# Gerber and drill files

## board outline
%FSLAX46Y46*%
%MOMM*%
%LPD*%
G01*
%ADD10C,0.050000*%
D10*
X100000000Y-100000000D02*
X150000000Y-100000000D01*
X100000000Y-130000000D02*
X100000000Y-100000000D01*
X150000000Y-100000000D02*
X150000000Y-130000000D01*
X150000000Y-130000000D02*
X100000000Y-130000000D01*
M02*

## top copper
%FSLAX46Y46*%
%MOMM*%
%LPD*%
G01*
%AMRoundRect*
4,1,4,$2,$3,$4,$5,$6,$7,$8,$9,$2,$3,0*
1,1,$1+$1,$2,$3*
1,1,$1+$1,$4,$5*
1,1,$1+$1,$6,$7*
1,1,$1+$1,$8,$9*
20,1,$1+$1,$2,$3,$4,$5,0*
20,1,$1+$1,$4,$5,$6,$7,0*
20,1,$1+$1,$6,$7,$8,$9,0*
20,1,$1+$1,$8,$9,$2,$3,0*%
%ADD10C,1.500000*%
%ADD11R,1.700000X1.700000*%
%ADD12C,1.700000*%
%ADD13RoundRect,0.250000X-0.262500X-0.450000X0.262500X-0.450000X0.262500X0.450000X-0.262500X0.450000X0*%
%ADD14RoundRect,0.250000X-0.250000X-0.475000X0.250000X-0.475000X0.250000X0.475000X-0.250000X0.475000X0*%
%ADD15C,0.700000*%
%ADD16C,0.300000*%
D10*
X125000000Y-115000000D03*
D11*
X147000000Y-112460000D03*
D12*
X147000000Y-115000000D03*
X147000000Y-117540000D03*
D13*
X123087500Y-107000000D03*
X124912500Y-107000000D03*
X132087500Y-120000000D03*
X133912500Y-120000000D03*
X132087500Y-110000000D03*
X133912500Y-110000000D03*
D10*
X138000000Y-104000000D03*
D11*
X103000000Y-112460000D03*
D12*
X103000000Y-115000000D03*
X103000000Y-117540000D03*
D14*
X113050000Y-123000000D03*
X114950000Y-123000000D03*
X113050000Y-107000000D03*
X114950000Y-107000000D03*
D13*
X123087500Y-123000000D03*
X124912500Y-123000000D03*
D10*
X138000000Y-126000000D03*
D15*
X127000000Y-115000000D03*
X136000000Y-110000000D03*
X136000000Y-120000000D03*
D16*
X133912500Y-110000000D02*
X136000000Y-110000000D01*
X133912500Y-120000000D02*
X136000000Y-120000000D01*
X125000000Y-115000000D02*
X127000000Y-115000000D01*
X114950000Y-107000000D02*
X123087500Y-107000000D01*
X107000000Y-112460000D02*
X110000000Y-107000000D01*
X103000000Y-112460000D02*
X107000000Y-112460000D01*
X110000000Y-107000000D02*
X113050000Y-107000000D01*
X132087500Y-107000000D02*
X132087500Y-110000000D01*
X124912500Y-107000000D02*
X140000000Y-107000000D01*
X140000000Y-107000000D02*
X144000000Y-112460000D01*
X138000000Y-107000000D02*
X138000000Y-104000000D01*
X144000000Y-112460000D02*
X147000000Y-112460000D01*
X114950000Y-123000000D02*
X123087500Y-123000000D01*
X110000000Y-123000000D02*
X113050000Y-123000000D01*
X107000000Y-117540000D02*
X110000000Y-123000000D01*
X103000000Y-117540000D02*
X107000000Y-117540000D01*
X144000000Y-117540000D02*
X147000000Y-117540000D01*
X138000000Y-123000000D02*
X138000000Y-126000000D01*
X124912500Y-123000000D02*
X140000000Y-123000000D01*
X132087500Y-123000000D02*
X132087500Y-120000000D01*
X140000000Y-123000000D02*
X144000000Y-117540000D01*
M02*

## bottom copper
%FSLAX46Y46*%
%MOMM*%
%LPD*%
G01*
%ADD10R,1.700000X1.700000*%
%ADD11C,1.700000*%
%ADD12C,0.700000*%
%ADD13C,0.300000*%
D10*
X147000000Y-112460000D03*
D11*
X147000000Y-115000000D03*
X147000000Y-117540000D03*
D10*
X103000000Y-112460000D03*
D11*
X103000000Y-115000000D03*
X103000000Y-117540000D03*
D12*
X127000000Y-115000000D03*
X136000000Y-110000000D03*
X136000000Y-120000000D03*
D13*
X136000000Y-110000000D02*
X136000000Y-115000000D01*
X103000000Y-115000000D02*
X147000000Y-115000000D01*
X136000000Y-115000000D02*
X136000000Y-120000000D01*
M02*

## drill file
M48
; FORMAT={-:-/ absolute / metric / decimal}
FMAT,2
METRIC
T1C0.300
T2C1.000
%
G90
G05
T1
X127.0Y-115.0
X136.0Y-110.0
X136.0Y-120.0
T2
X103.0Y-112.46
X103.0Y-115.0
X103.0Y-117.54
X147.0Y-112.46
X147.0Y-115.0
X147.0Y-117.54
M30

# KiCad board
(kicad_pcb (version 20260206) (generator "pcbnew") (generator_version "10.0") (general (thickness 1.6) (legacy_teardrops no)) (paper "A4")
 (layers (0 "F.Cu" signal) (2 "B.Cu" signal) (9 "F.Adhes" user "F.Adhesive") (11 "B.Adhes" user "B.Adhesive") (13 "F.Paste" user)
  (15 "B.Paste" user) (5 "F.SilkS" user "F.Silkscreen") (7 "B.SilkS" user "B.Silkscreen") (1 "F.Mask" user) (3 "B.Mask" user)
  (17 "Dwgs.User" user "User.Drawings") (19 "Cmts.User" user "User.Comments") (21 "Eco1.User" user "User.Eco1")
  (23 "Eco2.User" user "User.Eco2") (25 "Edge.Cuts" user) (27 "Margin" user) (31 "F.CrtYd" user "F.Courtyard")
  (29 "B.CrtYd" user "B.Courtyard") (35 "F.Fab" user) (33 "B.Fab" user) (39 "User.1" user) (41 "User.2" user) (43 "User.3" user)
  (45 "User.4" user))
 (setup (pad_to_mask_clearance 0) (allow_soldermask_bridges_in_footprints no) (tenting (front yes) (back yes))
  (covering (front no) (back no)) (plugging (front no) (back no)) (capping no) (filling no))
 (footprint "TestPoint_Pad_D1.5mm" (layer "F.Cu") (at 125 115)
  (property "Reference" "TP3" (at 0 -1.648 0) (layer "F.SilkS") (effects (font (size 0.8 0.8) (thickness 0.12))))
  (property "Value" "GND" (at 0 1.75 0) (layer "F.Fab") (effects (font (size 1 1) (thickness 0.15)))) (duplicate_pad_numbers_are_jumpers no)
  (pad "1" smd circle (at 0 0) (size 1.5 1.5) (layers "F.Cu" "F.Mask") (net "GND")))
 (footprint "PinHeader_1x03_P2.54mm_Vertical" (layer "F.Cu") (at 147 112.46)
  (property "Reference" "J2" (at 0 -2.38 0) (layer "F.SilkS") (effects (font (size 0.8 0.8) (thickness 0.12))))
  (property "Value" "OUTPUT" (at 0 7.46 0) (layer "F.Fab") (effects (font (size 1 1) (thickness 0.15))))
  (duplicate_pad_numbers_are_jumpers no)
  (pad "1" thru_hole rect (at 0 0) (size 1.7 1.7) (drill 1) (layers "*.Cu" "*.Mask") (remove_unused_layers no) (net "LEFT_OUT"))
  (pad "2" thru_hole circle (at 0 2.54) (size 1.7 1.7) (drill 1) (layers "*.Cu" "*.Mask") (remove_unused_layers no) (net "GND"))
  (pad "3" thru_hole circle (at 0 5.08) (size 1.7 1.7) (drill 1) (layers "*.Cu" "*.Mask") (remove_unused_layers no) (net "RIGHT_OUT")))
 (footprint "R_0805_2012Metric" (layer "F.Cu") (at 124 107)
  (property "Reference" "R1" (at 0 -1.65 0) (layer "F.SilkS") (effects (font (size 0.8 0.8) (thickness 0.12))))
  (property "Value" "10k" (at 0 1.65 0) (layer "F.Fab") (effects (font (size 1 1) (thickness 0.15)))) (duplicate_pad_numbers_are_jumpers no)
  (pad "1" smd roundrect (at -0.9125 0) (size 1.025 1.4) (layers "F.Cu" "F.Mask" "F.Paste") (roundrect_rratio 0.243902) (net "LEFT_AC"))
  (pad "2" smd roundrect (at 0.9125 0) (size 1.025 1.4) (layers "F.Cu" "F.Mask" "F.Paste") (roundrect_rratio 0.243902) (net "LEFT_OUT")))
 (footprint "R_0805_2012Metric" (layer "F.Cu") (at 133 120)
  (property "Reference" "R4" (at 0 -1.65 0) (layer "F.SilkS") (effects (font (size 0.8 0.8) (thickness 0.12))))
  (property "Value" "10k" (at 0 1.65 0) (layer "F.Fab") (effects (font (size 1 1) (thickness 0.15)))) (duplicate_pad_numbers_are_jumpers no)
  (pad "1" smd roundrect (at -0.9125 0) (size 1.025 1.4) (layers "F.Cu" "F.Mask" "F.Paste") (roundrect_rratio 0.243902) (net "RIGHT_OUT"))
  (pad "2" smd roundrect (at 0.9125 0) (size 1.025 1.4) (layers "F.Cu" "F.Mask" "F.Paste") (roundrect_rratio 0.243902) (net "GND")))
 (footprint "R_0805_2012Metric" (layer "F.Cu") (at 133 110)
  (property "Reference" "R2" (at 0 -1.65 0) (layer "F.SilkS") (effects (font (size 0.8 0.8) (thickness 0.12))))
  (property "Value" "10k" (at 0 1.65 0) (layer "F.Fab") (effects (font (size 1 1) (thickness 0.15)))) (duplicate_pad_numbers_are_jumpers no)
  (pad "1" smd roundrect (at -0.9125 0) (size 1.025 1.4) (layers "F.Cu" "F.Mask" "F.Paste") (roundrect_rratio 0.243902) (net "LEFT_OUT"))
  (pad "2" smd roundrect (at 0.9125 0) (size 1.025 1.4) (layers "F.Cu" "F.Mask" "F.Paste") (roundrect_rratio 0.243902) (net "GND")))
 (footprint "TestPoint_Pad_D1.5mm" (layer "F.Cu") (at 138 104)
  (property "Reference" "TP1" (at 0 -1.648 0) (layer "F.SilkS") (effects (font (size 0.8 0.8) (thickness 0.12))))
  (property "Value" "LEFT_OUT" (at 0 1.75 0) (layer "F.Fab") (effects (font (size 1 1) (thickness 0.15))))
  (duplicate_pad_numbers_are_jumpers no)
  (pad "1" smd circle (at 0 0) (size 1.5 1.5) (layers "F.Cu" "F.Mask") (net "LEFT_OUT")))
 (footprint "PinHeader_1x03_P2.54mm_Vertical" (layer "F.Cu") (at 103 112.46)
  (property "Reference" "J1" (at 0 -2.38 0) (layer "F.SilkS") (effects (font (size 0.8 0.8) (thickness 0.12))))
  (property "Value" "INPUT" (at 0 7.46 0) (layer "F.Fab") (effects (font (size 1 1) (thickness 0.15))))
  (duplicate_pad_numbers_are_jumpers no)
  (pad "1" thru_hole rect (at 0 0) (size 1.7 1.7) (drill 1) (layers "*.Cu" "*.Mask") (remove_unused_layers no) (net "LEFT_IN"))
  (pad "2" thru_hole circle (at 0 2.54) (size 1.7 1.7) (drill 1) (layers "*.Cu" "*.Mask") (remove_unused_layers no) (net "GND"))
  (pad "3" thru_hole circle (at 0 5.08) (size 1.7 1.7) (drill 1) (layers "*.Cu" "*.Mask") (remove_unused_layers no) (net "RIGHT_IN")))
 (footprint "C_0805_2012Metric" (layer "F.Cu") (at 114 123)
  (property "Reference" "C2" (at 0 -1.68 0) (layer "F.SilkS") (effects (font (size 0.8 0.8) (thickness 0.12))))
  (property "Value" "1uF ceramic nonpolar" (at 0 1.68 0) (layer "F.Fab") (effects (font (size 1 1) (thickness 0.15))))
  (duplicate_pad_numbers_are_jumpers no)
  (pad "1" smd roundrect (at -0.95 0) (size 1 1.45) (layers "F.Cu" "F.Mask" "F.Paste") (roundrect_rratio 0.25) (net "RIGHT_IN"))
  (pad "2" smd roundrect (at 0.95 0) (size 1 1.45) (layers "F.Cu" "F.Mask" "F.Paste") (roundrect_rratio 0.25) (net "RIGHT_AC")))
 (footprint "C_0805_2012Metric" (layer "F.Cu") (at 114 107)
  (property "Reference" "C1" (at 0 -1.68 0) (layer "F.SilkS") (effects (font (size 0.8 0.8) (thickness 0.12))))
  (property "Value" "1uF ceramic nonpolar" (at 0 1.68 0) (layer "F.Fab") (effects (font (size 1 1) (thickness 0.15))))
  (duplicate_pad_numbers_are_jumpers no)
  (pad "1" smd roundrect (at -0.95 0) (size 1 1.45) (layers "F.Cu" "F.Mask" "F.Paste") (roundrect_rratio 0.25) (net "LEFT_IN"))
  (pad "2" smd roundrect (at 0.95 0) (size 1 1.45) (layers "F.Cu" "F.Mask" "F.Paste") (roundrect_rratio 0.25) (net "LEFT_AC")))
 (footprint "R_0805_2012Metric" (layer "F.Cu") (at 124 123)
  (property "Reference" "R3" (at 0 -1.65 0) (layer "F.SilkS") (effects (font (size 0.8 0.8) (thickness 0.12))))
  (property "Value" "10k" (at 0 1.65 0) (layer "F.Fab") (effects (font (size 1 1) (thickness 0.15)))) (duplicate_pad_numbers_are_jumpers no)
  (pad "1" smd roundrect (at -0.9125 0) (size 1.025 1.4) (layers "F.Cu" "F.Mask" "F.Paste") (roundrect_rratio 0.243902) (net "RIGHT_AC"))
  (pad "2" smd roundrect (at 0.9125 0) (size 1.025 1.4) (layers "F.Cu" "F.Mask" "F.Paste") (roundrect_rratio 0.243902) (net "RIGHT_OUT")))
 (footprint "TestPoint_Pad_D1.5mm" (layer "F.Cu") (at 138 126)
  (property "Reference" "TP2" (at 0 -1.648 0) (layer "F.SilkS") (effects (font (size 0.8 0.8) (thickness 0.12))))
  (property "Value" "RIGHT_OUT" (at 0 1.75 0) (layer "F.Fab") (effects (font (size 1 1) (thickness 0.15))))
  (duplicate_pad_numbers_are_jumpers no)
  (pad "1" smd circle (at 0 0) (size 1.5 1.5) (layers "F.Cu" "F.Mask") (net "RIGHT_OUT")))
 (gr_line (start 100 100) (end 150 100) (stroke (width 0.05) (type default)) (layer "Edge.Cuts"))
 (gr_line (start 100 130) (end 100 100) (stroke (width 0.05) (type default)) (layer "Edge.Cuts"))
 (gr_line (start 150 100) (end 150 130) (stroke (width 0.05) (type default)) (layer "Edge.Cuts"))
 (gr_line (start 150 130) (end 100 130) (stroke (width 0.05) (type default)) (layer "Edge.Cuts"))
 (segment (start 133.9125 110) (end 136 110) (width 0.3) (layer "F.Cu") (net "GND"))
 (segment (start 133.9125 120) (end 136 120) (width 0.3) (layer "F.Cu") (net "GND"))
 (segment (start 125 115) (end 127 115) (width 0.3) (layer "F.Cu") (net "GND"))
 (via (at 127 115) (size 0.7) (drill 0.3) (layers "F.Cu" "B.Cu") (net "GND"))
 (via (at 136 110) (size 0.7) (drill 0.3) (layers "F.Cu" "B.Cu") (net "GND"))
 (via (at 136 120) (size 0.7) (drill 0.3) (layers "F.Cu" "B.Cu") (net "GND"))
 (segment (start 136 110) (end 136 115) (width 0.3) (layer "B.Cu") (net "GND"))
 (segment (start 103 115) (end 147 115) (width 0.3) (layer "B.Cu") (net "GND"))
 (segment (start 136 115) (end 136 120) (width 0.3) (layer "B.Cu") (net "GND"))
 (segment (start 114.95 107) (end 123.0875 107) (width 0.3) (layer "F.Cu") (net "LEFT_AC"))
 (segment (start 107 112.46) (end 110 107) (width 0.3) (layer "F.Cu") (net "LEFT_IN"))
 (segment (start 103 112.46) (end 107 112.46) (width 0.3) (layer "F.Cu") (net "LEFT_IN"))
 (segment (start 110 107) (end 113.05 107) (width 0.3) (layer "F.Cu") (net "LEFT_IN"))
 (segment (start 132.0875 107) (end 132.0875 110) (width 0.3) (layer "F.Cu") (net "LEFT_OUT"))
 (segment (start 124.9125 107) (end 140 107) (width 0.3) (layer "F.Cu") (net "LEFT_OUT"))
 (segment (start 140 107) (end 144 112.46) (width 0.3) (layer "F.Cu") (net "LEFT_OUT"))
 (segment (start 138 107) (end 138 104) (width 0.3) (layer "F.Cu") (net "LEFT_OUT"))
 (segment (start 144 112.46) (end 147 112.46) (width 0.3) (layer "F.Cu") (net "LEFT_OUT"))
 (segment (start 114.95 123) (end 123.0875 123) (width 0.3) (layer "F.Cu") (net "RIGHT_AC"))
 (segment (start 110 123) (end 113.05 123) (width 0.3) (layer "F.Cu") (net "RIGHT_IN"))
 (segment (start 107 117.54) (end 110 123) (width 0.3) (layer "F.Cu") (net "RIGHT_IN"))
 (segment (start 103 117.54) (end 107 117.54) (width 0.3) (layer "F.Cu") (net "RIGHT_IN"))
 (segment (start 144 117.54) (end 147 117.54) (width 0.3) (layer "F.Cu") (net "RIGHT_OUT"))
 (segment (start 138 123) (end 138 126) (width 0.3) (layer "F.Cu") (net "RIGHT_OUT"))
 (segment (start 124.9125 123) (end 140 123) (width 0.3) (layer "F.Cu") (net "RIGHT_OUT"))
 (segment (start 132.0875 123) (end 132.0875 120) (width 0.3) (layer "F.Cu") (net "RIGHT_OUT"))
 (segment (start 140 123) (end 144 117.54) (width 0.3) (layer "F.Cu") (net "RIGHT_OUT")))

